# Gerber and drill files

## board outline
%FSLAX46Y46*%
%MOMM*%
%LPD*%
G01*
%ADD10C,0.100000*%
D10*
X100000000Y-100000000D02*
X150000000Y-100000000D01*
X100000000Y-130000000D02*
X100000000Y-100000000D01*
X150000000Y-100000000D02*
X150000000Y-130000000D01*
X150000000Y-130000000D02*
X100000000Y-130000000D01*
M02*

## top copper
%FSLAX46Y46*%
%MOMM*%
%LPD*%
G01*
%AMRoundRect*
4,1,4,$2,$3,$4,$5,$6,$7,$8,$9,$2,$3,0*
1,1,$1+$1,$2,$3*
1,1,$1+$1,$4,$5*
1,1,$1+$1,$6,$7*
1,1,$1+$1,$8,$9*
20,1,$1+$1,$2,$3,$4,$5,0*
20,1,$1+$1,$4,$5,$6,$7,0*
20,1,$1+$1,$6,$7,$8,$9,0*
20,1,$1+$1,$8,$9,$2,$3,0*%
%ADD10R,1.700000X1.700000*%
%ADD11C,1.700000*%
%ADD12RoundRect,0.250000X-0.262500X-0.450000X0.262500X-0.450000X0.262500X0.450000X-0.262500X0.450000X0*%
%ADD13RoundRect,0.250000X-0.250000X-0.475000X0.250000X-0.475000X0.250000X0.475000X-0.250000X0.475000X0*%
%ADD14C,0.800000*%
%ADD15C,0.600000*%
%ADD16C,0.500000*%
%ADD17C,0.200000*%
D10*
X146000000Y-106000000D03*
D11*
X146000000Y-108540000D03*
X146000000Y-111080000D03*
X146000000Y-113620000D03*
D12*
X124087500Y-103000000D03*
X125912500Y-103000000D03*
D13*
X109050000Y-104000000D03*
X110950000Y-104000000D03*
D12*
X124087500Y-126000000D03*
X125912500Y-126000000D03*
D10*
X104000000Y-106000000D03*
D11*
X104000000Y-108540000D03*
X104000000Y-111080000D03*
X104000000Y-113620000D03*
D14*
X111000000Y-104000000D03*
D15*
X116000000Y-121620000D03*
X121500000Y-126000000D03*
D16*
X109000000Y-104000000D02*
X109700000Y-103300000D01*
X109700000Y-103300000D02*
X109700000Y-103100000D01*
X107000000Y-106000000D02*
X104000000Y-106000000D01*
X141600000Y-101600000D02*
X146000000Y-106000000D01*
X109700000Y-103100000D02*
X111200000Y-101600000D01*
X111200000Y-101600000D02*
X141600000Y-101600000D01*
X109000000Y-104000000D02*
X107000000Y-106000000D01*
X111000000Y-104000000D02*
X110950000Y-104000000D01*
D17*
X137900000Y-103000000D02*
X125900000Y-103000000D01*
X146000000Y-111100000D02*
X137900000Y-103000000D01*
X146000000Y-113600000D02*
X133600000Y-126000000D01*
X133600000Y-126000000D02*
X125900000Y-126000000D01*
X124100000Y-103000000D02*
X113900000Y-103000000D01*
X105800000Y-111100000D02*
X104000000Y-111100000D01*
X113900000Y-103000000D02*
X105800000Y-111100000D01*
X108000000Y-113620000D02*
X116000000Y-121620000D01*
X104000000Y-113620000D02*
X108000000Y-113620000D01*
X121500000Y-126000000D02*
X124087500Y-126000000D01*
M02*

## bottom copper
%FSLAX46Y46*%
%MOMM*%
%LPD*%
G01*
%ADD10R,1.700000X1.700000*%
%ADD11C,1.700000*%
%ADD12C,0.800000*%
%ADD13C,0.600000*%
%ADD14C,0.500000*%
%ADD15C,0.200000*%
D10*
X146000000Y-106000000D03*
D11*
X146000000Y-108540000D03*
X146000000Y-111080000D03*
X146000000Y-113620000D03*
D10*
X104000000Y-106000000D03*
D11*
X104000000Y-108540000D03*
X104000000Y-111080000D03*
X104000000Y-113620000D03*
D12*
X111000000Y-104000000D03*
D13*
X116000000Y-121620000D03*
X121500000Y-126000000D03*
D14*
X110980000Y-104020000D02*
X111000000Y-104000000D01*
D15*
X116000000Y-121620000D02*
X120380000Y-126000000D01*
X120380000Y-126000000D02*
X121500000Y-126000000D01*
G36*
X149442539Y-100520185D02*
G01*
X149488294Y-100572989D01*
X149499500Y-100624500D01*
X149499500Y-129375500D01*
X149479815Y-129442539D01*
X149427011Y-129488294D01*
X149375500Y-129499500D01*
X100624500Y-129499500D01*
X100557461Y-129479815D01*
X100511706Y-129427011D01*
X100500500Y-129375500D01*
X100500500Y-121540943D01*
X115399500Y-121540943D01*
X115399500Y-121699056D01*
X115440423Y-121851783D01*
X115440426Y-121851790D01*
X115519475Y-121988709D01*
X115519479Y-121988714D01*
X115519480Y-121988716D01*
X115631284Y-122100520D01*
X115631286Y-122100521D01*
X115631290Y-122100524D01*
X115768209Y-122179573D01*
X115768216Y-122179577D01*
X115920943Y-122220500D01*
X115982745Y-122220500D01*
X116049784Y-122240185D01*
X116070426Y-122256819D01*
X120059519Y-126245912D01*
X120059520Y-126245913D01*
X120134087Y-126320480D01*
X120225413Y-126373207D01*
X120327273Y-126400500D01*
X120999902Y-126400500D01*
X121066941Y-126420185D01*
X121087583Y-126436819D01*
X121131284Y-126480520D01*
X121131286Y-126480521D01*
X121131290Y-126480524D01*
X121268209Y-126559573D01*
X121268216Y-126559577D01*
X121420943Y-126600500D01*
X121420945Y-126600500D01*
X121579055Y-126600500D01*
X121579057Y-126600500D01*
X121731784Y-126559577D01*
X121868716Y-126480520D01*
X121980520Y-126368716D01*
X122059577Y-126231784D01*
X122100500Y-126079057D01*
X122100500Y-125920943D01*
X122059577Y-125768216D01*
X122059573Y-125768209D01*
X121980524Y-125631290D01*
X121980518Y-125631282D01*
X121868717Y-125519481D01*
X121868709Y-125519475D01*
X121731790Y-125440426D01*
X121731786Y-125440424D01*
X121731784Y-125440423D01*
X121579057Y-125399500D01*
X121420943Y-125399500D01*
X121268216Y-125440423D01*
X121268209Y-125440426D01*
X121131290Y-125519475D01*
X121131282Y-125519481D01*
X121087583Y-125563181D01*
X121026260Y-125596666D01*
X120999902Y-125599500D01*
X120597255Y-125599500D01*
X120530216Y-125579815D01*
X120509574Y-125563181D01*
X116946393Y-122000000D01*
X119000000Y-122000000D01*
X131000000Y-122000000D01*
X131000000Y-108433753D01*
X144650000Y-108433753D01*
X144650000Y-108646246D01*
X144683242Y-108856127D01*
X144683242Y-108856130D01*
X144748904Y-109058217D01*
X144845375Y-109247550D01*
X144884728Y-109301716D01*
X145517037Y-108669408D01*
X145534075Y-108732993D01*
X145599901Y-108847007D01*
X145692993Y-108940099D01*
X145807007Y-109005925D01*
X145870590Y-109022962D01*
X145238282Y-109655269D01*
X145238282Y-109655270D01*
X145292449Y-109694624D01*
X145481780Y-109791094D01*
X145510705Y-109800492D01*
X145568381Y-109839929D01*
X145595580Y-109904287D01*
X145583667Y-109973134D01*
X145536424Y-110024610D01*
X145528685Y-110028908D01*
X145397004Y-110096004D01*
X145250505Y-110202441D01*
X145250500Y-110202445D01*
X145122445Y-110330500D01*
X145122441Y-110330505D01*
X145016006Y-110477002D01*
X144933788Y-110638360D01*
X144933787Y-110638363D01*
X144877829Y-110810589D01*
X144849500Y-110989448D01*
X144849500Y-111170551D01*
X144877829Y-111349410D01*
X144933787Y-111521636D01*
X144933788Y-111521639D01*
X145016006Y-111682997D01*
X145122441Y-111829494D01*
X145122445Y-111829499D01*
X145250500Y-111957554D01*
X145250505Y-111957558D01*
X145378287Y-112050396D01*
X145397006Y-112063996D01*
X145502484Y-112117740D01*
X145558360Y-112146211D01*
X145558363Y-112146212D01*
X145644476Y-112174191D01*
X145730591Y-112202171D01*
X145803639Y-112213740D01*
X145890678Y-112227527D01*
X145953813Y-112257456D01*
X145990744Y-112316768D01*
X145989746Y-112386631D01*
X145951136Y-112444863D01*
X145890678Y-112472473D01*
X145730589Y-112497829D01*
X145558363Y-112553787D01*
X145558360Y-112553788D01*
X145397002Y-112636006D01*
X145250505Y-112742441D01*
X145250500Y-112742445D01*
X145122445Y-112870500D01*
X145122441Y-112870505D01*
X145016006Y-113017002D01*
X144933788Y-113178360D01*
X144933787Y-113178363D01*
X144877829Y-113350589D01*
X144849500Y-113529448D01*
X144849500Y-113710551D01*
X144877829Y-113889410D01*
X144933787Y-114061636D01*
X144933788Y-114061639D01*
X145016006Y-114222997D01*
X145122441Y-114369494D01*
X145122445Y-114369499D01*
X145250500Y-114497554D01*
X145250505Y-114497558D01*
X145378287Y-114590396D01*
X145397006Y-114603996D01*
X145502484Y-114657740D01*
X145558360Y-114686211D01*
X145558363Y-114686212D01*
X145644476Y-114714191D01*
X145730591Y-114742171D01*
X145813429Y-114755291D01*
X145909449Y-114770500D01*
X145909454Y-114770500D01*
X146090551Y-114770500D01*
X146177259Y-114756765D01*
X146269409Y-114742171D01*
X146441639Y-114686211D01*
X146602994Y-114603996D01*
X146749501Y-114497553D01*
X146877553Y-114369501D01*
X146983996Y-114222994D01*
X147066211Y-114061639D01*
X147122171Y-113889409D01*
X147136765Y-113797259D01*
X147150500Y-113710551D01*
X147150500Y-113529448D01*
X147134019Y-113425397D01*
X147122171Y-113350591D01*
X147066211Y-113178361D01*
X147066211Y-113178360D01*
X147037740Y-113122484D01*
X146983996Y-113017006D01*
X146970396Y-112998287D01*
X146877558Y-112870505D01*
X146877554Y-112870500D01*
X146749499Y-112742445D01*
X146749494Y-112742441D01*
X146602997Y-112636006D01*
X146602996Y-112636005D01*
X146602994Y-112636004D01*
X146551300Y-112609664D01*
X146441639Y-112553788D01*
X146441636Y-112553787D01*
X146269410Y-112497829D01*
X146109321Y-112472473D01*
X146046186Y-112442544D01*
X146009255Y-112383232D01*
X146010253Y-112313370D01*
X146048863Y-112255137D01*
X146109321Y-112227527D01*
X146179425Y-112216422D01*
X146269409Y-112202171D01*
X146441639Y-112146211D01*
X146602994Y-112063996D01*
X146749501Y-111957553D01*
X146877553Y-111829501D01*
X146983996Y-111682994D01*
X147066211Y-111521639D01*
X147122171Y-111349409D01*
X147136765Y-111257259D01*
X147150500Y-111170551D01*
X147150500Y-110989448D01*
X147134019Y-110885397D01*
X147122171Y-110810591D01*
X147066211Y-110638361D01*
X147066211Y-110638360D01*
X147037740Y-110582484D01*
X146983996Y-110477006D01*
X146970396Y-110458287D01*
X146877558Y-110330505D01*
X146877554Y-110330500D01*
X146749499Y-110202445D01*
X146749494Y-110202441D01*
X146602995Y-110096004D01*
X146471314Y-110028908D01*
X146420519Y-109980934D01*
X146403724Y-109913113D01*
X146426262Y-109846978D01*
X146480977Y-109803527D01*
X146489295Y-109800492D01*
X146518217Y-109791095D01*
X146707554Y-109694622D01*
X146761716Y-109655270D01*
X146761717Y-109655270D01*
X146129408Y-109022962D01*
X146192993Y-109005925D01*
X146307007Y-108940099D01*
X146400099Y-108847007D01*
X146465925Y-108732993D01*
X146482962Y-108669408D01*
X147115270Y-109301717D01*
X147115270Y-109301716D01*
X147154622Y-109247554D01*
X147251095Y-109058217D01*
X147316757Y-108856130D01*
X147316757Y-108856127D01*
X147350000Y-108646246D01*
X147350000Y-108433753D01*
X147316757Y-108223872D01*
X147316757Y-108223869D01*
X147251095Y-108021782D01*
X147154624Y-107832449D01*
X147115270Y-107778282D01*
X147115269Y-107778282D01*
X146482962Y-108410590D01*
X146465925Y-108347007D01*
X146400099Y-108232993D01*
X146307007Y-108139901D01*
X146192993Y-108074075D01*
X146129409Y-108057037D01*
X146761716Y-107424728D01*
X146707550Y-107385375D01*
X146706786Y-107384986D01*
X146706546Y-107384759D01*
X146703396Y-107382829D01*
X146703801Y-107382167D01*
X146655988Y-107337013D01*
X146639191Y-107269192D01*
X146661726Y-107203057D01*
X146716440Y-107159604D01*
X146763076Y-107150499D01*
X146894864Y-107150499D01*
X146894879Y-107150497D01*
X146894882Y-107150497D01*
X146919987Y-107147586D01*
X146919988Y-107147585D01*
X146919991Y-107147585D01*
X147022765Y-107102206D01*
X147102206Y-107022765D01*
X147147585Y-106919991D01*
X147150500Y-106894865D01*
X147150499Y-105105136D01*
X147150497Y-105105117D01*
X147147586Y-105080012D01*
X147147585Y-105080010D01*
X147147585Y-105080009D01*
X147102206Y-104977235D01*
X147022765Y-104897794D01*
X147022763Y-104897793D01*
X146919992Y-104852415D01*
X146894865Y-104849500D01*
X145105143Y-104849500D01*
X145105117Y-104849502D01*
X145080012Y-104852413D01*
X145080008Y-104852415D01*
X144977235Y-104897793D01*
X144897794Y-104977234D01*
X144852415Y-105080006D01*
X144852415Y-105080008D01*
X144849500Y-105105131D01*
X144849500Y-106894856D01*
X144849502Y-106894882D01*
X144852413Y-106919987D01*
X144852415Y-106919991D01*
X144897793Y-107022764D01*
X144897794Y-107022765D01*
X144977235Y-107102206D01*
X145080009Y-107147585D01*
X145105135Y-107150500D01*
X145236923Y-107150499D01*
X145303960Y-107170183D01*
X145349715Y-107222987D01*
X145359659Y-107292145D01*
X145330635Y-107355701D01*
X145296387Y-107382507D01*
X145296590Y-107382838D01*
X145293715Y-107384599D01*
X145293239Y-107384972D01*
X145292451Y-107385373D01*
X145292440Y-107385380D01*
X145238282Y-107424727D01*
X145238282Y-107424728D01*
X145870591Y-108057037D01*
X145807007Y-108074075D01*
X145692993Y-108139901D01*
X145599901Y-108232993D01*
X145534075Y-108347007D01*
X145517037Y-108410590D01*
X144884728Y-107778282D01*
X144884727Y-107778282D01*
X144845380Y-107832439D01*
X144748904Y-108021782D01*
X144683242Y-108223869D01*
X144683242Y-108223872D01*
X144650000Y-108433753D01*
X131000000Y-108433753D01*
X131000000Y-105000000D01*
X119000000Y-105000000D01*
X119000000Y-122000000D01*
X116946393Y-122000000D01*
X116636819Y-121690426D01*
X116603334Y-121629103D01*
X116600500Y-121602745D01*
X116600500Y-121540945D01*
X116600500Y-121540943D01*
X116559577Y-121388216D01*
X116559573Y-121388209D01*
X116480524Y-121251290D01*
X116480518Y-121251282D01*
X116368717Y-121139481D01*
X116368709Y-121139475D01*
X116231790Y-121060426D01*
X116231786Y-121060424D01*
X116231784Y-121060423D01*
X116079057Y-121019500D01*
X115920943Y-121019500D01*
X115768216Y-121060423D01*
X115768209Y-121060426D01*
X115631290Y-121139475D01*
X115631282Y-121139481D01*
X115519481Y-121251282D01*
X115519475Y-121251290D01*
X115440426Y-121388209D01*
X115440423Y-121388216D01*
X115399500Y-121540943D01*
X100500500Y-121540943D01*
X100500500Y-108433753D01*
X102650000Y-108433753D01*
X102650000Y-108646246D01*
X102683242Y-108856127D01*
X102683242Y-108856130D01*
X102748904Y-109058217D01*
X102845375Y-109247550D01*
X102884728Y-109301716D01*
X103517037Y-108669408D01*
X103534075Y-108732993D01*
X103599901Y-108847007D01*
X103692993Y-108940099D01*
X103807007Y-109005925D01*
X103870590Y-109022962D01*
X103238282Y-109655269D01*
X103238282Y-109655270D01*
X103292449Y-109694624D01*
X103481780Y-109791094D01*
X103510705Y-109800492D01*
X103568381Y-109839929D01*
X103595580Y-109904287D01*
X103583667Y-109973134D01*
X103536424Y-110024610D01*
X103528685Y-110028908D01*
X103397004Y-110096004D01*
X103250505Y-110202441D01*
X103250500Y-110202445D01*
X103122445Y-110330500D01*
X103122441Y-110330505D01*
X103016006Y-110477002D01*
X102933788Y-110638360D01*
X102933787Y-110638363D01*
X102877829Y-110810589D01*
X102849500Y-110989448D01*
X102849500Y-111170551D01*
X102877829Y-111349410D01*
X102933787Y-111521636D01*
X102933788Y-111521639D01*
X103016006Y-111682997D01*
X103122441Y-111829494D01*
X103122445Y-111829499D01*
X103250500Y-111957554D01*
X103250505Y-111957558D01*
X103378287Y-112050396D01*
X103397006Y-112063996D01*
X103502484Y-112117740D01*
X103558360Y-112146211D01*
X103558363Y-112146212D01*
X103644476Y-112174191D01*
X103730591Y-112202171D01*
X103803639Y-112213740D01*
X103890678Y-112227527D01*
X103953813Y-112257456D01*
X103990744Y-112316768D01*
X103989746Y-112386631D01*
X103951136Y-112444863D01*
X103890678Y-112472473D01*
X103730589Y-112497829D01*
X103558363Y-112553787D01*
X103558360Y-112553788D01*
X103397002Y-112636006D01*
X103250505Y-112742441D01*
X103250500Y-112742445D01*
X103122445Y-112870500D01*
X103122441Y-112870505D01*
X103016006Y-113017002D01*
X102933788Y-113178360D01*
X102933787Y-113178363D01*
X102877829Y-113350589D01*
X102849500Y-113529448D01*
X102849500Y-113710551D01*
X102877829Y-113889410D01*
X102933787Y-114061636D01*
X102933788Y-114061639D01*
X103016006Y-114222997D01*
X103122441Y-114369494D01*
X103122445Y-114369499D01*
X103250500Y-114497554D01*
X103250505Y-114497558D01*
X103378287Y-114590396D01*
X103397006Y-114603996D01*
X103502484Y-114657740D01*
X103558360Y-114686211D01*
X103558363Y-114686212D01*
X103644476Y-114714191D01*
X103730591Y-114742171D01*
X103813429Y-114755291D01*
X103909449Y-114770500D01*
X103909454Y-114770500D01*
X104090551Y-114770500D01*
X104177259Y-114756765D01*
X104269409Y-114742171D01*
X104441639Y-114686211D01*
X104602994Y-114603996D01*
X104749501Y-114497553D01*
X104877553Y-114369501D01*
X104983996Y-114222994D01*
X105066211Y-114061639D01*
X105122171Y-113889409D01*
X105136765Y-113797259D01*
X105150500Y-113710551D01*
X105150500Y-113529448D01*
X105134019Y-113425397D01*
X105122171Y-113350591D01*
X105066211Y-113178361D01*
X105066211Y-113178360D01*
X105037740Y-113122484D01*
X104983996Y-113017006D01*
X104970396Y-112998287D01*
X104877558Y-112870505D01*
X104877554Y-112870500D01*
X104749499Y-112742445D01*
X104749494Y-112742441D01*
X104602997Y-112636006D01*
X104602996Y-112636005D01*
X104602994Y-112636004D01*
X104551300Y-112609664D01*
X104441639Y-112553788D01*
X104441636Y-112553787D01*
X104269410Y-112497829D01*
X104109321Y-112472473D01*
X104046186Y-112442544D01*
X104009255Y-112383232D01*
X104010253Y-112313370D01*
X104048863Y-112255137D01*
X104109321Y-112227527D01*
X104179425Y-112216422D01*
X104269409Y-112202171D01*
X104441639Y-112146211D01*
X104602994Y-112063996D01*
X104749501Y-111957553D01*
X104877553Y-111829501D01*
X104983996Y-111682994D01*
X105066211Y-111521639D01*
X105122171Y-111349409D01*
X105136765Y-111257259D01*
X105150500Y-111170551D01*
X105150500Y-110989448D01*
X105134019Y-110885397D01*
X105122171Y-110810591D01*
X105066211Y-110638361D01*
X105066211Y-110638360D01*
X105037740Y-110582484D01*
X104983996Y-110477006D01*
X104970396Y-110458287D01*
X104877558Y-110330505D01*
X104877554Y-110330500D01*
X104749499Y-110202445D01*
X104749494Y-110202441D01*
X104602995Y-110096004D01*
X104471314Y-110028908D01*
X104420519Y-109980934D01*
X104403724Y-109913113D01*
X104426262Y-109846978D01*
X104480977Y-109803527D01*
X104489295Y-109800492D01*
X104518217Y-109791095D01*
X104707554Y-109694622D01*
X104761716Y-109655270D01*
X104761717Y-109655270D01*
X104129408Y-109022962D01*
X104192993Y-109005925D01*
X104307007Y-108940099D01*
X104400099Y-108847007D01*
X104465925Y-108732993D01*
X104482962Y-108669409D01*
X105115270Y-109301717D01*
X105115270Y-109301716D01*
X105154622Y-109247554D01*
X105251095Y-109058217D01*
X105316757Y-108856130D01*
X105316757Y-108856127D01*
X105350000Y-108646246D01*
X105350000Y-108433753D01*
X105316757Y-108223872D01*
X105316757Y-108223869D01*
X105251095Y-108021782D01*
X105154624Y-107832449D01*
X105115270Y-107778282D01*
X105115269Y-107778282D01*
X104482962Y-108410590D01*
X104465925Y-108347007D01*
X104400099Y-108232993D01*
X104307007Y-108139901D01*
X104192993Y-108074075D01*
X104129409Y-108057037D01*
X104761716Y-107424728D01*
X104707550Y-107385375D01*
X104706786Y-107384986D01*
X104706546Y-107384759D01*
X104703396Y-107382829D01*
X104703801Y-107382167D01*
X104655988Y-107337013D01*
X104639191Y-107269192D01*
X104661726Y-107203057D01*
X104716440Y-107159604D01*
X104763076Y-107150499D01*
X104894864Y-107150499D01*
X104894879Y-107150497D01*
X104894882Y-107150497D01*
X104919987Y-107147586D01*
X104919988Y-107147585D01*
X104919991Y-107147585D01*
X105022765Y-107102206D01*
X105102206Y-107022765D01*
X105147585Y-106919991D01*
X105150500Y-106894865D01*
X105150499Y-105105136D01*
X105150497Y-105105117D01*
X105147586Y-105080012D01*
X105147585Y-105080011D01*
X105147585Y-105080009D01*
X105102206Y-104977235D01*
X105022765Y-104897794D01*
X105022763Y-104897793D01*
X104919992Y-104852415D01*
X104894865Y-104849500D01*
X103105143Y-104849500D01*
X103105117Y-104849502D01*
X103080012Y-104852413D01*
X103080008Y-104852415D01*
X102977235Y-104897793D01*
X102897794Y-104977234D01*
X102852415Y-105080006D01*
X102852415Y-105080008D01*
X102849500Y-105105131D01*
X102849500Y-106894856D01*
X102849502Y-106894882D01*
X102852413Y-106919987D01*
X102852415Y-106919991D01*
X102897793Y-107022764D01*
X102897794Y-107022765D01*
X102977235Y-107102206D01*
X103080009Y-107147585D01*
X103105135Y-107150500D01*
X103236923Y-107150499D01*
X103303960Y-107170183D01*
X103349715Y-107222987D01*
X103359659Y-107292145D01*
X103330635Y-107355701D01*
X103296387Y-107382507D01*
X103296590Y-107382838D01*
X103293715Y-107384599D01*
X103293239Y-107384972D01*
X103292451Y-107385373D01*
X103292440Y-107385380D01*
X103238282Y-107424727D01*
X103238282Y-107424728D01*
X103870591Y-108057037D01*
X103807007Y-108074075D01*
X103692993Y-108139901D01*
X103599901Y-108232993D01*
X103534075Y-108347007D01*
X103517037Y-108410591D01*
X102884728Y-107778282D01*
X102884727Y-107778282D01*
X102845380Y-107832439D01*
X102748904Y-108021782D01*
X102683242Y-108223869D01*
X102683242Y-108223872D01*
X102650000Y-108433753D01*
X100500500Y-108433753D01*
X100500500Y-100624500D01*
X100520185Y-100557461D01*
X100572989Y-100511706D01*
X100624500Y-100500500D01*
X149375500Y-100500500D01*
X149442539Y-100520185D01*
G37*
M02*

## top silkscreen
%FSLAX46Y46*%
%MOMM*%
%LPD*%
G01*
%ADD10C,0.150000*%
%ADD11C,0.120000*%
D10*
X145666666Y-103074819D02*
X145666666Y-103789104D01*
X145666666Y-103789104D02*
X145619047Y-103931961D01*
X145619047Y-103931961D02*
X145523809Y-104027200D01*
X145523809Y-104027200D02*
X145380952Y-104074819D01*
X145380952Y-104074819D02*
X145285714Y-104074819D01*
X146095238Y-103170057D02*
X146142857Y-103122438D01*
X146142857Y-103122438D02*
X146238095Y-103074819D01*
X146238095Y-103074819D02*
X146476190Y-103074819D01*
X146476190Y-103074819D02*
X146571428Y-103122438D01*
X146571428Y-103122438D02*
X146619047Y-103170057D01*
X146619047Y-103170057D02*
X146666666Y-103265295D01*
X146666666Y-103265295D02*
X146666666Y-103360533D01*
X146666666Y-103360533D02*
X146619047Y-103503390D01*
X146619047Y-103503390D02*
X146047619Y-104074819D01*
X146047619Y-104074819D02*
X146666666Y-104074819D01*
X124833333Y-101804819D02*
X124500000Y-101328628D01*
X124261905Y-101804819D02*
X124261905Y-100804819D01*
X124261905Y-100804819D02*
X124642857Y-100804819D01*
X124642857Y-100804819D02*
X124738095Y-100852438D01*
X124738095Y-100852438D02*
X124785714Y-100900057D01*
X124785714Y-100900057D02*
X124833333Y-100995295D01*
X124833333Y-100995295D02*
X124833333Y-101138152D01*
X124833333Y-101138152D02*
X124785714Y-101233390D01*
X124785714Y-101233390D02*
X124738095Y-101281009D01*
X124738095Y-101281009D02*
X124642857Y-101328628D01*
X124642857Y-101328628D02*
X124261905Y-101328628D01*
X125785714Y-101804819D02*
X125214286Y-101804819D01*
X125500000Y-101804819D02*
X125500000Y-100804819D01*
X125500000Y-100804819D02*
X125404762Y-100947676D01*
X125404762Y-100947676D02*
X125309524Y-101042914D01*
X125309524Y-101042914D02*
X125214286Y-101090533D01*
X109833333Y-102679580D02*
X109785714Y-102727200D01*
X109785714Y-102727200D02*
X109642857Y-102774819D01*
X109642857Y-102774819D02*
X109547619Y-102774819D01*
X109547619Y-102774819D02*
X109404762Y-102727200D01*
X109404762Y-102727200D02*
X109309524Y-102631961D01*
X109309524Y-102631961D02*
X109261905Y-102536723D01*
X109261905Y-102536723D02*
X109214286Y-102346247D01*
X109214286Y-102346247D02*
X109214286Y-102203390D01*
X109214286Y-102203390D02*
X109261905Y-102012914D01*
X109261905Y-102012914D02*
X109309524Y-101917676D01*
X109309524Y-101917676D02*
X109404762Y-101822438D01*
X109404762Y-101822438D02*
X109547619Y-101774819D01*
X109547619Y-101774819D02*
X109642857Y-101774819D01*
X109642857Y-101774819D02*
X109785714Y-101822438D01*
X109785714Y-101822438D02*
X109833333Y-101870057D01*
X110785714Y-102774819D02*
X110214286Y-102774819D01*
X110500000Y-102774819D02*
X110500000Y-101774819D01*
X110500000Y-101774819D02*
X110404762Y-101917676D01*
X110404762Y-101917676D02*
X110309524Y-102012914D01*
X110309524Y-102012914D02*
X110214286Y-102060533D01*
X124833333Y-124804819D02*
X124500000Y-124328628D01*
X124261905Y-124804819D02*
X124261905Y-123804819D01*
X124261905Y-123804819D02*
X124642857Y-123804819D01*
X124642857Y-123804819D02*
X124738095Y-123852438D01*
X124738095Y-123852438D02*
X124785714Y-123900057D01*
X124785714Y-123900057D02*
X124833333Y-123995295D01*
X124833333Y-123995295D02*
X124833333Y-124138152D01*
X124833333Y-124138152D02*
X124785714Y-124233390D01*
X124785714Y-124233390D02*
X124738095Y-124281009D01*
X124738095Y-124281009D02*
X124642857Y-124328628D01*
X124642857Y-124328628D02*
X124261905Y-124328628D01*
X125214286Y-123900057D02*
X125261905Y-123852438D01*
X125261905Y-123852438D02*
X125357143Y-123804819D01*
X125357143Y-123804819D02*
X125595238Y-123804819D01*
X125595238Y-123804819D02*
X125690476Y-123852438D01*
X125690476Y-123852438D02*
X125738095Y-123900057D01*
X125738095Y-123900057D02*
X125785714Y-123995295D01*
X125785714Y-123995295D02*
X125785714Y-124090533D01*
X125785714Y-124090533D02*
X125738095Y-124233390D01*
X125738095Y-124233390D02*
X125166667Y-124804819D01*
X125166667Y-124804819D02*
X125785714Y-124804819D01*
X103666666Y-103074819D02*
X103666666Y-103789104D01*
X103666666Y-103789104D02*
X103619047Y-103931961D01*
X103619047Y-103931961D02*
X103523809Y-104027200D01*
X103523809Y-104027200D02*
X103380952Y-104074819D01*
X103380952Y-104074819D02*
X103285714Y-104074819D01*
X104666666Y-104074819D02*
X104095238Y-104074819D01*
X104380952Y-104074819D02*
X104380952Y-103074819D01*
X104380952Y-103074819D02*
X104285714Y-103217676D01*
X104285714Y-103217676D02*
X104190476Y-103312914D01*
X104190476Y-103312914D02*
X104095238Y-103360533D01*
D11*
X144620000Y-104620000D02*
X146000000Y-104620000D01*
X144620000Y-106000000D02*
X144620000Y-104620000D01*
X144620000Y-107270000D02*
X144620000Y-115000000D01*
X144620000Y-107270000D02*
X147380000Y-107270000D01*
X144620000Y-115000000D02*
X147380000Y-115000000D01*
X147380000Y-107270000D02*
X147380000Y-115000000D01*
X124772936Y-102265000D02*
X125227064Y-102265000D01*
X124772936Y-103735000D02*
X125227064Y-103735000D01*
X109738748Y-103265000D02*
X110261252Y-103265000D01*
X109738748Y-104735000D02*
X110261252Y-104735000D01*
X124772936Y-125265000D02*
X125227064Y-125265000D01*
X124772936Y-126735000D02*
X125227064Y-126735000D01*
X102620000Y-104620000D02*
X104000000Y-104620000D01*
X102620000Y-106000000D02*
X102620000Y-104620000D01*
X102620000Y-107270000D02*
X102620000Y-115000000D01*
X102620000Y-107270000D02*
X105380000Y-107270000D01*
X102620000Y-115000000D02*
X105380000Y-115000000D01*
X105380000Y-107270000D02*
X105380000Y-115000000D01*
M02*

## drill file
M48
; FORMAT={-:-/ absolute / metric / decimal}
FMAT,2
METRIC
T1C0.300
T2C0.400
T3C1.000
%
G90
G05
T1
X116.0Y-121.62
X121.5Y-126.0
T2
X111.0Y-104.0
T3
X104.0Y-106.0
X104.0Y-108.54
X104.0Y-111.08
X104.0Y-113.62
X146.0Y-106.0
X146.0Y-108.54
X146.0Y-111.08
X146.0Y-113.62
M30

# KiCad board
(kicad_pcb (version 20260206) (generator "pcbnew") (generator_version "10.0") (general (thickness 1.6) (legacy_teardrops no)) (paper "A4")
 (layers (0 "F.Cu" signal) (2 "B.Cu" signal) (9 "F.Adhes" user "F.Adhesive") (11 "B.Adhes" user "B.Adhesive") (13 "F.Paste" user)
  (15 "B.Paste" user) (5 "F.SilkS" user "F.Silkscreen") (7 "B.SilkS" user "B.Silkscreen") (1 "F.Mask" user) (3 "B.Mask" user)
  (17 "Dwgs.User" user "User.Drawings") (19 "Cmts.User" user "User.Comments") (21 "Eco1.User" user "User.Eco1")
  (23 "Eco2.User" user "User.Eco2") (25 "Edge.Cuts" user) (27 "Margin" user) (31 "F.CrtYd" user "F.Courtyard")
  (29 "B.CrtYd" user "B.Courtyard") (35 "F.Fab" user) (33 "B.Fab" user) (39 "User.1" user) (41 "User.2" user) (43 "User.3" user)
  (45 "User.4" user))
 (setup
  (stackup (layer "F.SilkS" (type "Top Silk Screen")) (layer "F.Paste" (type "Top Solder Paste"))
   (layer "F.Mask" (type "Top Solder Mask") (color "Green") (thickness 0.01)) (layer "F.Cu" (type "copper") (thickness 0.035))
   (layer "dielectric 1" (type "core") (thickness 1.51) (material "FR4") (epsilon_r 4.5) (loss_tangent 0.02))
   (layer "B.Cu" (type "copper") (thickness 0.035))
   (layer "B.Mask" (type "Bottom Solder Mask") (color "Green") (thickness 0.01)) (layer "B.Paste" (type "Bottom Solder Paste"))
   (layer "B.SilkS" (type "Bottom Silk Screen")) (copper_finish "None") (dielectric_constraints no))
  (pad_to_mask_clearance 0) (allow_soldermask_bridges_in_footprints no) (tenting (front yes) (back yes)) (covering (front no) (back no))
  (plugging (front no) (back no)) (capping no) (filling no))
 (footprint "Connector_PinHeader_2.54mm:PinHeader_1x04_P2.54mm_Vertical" (layer "F.Cu") (at 146 106)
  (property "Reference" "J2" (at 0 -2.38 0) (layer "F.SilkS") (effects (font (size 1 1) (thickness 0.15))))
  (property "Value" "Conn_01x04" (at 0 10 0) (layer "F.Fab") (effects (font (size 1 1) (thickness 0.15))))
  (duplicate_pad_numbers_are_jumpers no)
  (fp_line (start -1.38 -1.38) (end 0 -1.38) (stroke (width 0.12) (type solid)) (layer "F.SilkS"))
  (fp_line (start -1.38 0) (end -1.38 -1.38) (stroke (width 0.12) (type solid)) (layer "F.SilkS"))
  (fp_line (start -1.38 1.27) (end -1.38 9) (stroke (width 0.12) (type solid)) (layer "F.SilkS"))
  (fp_line (start -1.38 1.27) (end 1.38 1.27) (stroke (width 0.12) (type solid)) (layer "F.SilkS"))
  (fp_line (start -1.38 9) (end 1.38 9) (stroke (width 0.12) (type solid)) (layer "F.SilkS"))
  (fp_line (start 1.38 1.27) (end 1.38 9) (stroke (width 0.12) (type solid)) (layer "F.SilkS"))
  (pad "1" thru_hole rect (at 0 0) (size 1.7 1.7) (drill 1) (layers "*.Cu" "*.Mask") (remove_unused_layers no) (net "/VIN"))
  (pad "2" thru_hole circle (at 0 2.54) (size 1.7 1.7) (drill 1) (layers "*.Cu" "*.Mask") (remove_unused_layers no) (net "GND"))
  (pad "3" thru_hole circle (at 0 5.08) (size 1.7 1.7) (drill 1) (layers "*.Cu" "*.Mask") (remove_unused_layers no) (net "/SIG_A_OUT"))
  (pad "4" thru_hole circle (at 0 7.62) (size 1.7 1.7) (drill 1) (layers "*.Cu" "*.Mask") (remove_unused_layers no) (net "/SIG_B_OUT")))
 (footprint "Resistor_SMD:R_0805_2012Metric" (layer "F.Cu") (at 125 103)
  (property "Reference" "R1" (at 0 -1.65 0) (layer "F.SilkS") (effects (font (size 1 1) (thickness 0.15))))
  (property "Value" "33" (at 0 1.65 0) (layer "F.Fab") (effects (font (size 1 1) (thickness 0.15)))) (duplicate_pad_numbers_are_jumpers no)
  (fp_line (start -0.227064 -0.735) (end 0.227064 -0.735) (stroke (width 0.12) (type solid)) (layer "F.SilkS"))
  (fp_line (start -0.227064 0.735) (end 0.227064 0.735) (stroke (width 0.12) (type solid)) (layer "F.SilkS"))
  (pad "1" smd roundrect (at -0.9125 0) (size 1.025 1.4) (layers "F.Cu" "F.Mask" "F.Paste") (roundrect_rratio 0.243902) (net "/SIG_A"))
  (pad "2" smd roundrect (at 0.9125 0) (size 1.025 1.4) (layers "F.Cu" "F.Mask" "F.Paste") (roundrect_rratio 0.243902) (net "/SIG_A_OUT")))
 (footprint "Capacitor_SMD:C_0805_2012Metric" (layer "F.Cu") (at 110 104)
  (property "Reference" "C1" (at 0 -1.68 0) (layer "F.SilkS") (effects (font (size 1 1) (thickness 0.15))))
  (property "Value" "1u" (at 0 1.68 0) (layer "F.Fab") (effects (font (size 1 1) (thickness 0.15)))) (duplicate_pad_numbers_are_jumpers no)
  (fp_line (start -0.261252 -0.735) (end 0.261252 -0.735) (stroke (width 0.12) (type solid)) (layer "F.SilkS"))
  (fp_line (start -0.261252 0.735) (end 0.261252 0.735) (stroke (width 0.12) (type solid)) (layer "F.SilkS"))
  (pad "1" smd roundrect (at -0.95 0) (size 1 1.45) (layers "F.Cu" "F.Mask" "F.Paste") (roundrect_rratio 0.25) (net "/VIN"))
  (pad "2" smd roundrect (at 0.95 0) (size 1 1.45) (layers "F.Cu" "F.Mask" "F.Paste") (roundrect_rratio 0.25) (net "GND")))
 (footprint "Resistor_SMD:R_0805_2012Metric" (layer "F.Cu") (at 125 126)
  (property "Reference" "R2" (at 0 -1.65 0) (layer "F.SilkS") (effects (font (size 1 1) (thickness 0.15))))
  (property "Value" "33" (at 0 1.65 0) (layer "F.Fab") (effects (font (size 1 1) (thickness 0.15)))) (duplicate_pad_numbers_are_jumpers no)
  (fp_line (start -0.227064 -0.735) (end 0.227064 -0.735) (stroke (width 0.12) (type solid)) (layer "F.SilkS"))
  (fp_line (start -0.227064 0.735) (end 0.227064 0.735) (stroke (width 0.12) (type solid)) (layer "F.SilkS"))
  (pad "1" smd roundrect (at -0.9125 0) (size 1.025 1.4) (layers "F.Cu" "F.Mask" "F.Paste") (roundrect_rratio 0.243902) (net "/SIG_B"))
  (pad "2" smd roundrect (at 0.9125 0) (size 1.025 1.4) (layers "F.Cu" "F.Mask" "F.Paste") (roundrect_rratio 0.243902) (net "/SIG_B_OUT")))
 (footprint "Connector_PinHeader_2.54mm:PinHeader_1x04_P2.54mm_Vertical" (layer "F.Cu") (at 104 106)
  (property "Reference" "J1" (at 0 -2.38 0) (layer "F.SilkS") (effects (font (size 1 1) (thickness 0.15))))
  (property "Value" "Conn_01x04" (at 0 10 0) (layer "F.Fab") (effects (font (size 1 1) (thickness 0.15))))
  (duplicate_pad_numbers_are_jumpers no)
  (fp_line (start -1.38 -1.38) (end 0 -1.38) (stroke (width 0.12) (type solid)) (layer "F.SilkS"))
  (fp_line (start -1.38 0) (end -1.38 -1.38) (stroke (width 0.12) (type solid)) (layer "F.SilkS"))
  (fp_line (start -1.38 1.27) (end -1.38 9) (stroke (width 0.12) (type solid)) (layer "F.SilkS"))
  (fp_line (start -1.38 1.27) (end 1.38 1.27) (stroke (width 0.12) (type solid)) (layer "F.SilkS"))
  (fp_line (start -1.38 9) (end 1.38 9) (stroke (width 0.12) (type solid)) (layer "F.SilkS"))
  (fp_line (start 1.38 1.27) (end 1.38 9) (stroke (width 0.12) (type solid)) (layer "F.SilkS"))
  (pad "1" thru_hole rect (at 0 0) (size 1.7 1.7) (drill 1) (layers "*.Cu" "*.Mask") (remove_unused_layers no) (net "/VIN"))
  (pad "2" thru_hole circle (at 0 2.54) (size 1.7 1.7) (drill 1) (layers "*.Cu" "*.Mask") (remove_unused_layers no) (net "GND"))
  (pad "3" thru_hole circle (at 0 5.08) (size 1.7 1.7) (drill 1) (layers "*.Cu" "*.Mask") (remove_unused_layers no) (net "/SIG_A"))
  (pad "4" thru_hole circle (at 0 7.62) (size 1.7 1.7) (drill 1) (layers "*.Cu" "*.Mask") (remove_unused_layers no) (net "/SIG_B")))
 (gr_line (start 100 100) (end 150 100) (stroke (width 0.1) (type default)) (layer "Edge.Cuts"))
 (gr_line (start 100 130) (end 100 100) (stroke (width 0.1) (type default)) (layer "Edge.Cuts"))
 (gr_line (start 150 100) (end 150 130) (stroke (width 0.1) (type default)) (layer "Edge.Cuts"))
 (gr_line (start 150 130) (end 100 130) (stroke (width 0.1) (type default)) (layer "Edge.Cuts"))
 (segment (start 109 104) (end 109.7 103.3) (width 0.5) (layer "F.Cu") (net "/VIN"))
 (segment (start 109.7 103.3) (end 109.7 103.1) (width 0.5) (layer "F.Cu") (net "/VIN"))
 (segment (start 107 106) (end 104 106) (width 0.5) (layer "F.Cu") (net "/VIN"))
 (segment (start 141.6 101.6) (end 146 106) (width 0.5) (layer "F.Cu") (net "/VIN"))
 (segment (start 109.7 103.1) (end 111.2 101.6) (width 0.5) (layer "F.Cu") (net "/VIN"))
 (segment (start 111.2 101.6) (end 141.6 101.6) (width 0.5) (layer "F.Cu") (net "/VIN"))
 (segment (start 109 104) (end 107 106) (width 0.5) (layer "F.Cu") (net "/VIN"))
 (segment (start 111 104) (end 110.95 104) (width 0.5) (layer "F.Cu") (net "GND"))
 (via (at 111 104) (size 0.8) (drill 0.4) (layers "F.Cu" "B.Cu") (capping yes) (filling yes) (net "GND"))
 (segment (start 110.98 104.02) (end 111 104) (width 0.5) (layer "B.Cu") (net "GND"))
 (segment (start 137.9 103) (end 125.9 103) (width 0.2) (layer "F.Cu") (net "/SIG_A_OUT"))
 (segment (start 146 111.1) (end 137.9 103) (width 0.2) (layer "F.Cu") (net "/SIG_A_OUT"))
 (segment (start 146 113.6) (end 133.6 126) (width 0.2) (layer "F.Cu") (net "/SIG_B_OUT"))
 (segment (start 133.6 126) (end 125.9 126) (width 0.2) (layer "F.Cu") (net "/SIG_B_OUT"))
 (segment (start 124.1 103) (end 113.9 103) (width 0.2) (layer "F.Cu") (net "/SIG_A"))
 (segment (start 105.8 111.1) (end 104 111.1) (width 0.2) (layer "F.Cu") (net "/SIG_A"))
 (segment (start 113.9 103) (end 105.8 111.1) (width 0.2) (layer "F.Cu") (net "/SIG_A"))
 (segment (start 108 113.62) (end 116 121.62) (width 0.2) (locked yes) (layer "F.Cu") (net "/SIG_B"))
 (segment (start 104 113.62) (end 108 113.62) (width 0.2) (locked yes) (layer "F.Cu") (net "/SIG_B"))
 (segment (start 121.5 126) (end 124.0875 126) (width 0.2) (locked yes) (layer "F.Cu") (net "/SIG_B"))
 (via (at 116 121.62) (size 0.6) (drill 0.3) (layers "F.Cu" "B.Cu") (locked yes) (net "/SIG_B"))
 (via (at 121.5 126) (size 0.6) (drill 0.3) (layers "F.Cu" "B.Cu") (locked yes) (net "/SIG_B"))
 (segment (start 116 121.62) (end 120.38 126) (width 0.2) (locked yes) (layer "B.Cu") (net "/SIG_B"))
 (segment (start 120.38 126) (end 121.5 126) (width 0.2) (locked yes) (layer "B.Cu") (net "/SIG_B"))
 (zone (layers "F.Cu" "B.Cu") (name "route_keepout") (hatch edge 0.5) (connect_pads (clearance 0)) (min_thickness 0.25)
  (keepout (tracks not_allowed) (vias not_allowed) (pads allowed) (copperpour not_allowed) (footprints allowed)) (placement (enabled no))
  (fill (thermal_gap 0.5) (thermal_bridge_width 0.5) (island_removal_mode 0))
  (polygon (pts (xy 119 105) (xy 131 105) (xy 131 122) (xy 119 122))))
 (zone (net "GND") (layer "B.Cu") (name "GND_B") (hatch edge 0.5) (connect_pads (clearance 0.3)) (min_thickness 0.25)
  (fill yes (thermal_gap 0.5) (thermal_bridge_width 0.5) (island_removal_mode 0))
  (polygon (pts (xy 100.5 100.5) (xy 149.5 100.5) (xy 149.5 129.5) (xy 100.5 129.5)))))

